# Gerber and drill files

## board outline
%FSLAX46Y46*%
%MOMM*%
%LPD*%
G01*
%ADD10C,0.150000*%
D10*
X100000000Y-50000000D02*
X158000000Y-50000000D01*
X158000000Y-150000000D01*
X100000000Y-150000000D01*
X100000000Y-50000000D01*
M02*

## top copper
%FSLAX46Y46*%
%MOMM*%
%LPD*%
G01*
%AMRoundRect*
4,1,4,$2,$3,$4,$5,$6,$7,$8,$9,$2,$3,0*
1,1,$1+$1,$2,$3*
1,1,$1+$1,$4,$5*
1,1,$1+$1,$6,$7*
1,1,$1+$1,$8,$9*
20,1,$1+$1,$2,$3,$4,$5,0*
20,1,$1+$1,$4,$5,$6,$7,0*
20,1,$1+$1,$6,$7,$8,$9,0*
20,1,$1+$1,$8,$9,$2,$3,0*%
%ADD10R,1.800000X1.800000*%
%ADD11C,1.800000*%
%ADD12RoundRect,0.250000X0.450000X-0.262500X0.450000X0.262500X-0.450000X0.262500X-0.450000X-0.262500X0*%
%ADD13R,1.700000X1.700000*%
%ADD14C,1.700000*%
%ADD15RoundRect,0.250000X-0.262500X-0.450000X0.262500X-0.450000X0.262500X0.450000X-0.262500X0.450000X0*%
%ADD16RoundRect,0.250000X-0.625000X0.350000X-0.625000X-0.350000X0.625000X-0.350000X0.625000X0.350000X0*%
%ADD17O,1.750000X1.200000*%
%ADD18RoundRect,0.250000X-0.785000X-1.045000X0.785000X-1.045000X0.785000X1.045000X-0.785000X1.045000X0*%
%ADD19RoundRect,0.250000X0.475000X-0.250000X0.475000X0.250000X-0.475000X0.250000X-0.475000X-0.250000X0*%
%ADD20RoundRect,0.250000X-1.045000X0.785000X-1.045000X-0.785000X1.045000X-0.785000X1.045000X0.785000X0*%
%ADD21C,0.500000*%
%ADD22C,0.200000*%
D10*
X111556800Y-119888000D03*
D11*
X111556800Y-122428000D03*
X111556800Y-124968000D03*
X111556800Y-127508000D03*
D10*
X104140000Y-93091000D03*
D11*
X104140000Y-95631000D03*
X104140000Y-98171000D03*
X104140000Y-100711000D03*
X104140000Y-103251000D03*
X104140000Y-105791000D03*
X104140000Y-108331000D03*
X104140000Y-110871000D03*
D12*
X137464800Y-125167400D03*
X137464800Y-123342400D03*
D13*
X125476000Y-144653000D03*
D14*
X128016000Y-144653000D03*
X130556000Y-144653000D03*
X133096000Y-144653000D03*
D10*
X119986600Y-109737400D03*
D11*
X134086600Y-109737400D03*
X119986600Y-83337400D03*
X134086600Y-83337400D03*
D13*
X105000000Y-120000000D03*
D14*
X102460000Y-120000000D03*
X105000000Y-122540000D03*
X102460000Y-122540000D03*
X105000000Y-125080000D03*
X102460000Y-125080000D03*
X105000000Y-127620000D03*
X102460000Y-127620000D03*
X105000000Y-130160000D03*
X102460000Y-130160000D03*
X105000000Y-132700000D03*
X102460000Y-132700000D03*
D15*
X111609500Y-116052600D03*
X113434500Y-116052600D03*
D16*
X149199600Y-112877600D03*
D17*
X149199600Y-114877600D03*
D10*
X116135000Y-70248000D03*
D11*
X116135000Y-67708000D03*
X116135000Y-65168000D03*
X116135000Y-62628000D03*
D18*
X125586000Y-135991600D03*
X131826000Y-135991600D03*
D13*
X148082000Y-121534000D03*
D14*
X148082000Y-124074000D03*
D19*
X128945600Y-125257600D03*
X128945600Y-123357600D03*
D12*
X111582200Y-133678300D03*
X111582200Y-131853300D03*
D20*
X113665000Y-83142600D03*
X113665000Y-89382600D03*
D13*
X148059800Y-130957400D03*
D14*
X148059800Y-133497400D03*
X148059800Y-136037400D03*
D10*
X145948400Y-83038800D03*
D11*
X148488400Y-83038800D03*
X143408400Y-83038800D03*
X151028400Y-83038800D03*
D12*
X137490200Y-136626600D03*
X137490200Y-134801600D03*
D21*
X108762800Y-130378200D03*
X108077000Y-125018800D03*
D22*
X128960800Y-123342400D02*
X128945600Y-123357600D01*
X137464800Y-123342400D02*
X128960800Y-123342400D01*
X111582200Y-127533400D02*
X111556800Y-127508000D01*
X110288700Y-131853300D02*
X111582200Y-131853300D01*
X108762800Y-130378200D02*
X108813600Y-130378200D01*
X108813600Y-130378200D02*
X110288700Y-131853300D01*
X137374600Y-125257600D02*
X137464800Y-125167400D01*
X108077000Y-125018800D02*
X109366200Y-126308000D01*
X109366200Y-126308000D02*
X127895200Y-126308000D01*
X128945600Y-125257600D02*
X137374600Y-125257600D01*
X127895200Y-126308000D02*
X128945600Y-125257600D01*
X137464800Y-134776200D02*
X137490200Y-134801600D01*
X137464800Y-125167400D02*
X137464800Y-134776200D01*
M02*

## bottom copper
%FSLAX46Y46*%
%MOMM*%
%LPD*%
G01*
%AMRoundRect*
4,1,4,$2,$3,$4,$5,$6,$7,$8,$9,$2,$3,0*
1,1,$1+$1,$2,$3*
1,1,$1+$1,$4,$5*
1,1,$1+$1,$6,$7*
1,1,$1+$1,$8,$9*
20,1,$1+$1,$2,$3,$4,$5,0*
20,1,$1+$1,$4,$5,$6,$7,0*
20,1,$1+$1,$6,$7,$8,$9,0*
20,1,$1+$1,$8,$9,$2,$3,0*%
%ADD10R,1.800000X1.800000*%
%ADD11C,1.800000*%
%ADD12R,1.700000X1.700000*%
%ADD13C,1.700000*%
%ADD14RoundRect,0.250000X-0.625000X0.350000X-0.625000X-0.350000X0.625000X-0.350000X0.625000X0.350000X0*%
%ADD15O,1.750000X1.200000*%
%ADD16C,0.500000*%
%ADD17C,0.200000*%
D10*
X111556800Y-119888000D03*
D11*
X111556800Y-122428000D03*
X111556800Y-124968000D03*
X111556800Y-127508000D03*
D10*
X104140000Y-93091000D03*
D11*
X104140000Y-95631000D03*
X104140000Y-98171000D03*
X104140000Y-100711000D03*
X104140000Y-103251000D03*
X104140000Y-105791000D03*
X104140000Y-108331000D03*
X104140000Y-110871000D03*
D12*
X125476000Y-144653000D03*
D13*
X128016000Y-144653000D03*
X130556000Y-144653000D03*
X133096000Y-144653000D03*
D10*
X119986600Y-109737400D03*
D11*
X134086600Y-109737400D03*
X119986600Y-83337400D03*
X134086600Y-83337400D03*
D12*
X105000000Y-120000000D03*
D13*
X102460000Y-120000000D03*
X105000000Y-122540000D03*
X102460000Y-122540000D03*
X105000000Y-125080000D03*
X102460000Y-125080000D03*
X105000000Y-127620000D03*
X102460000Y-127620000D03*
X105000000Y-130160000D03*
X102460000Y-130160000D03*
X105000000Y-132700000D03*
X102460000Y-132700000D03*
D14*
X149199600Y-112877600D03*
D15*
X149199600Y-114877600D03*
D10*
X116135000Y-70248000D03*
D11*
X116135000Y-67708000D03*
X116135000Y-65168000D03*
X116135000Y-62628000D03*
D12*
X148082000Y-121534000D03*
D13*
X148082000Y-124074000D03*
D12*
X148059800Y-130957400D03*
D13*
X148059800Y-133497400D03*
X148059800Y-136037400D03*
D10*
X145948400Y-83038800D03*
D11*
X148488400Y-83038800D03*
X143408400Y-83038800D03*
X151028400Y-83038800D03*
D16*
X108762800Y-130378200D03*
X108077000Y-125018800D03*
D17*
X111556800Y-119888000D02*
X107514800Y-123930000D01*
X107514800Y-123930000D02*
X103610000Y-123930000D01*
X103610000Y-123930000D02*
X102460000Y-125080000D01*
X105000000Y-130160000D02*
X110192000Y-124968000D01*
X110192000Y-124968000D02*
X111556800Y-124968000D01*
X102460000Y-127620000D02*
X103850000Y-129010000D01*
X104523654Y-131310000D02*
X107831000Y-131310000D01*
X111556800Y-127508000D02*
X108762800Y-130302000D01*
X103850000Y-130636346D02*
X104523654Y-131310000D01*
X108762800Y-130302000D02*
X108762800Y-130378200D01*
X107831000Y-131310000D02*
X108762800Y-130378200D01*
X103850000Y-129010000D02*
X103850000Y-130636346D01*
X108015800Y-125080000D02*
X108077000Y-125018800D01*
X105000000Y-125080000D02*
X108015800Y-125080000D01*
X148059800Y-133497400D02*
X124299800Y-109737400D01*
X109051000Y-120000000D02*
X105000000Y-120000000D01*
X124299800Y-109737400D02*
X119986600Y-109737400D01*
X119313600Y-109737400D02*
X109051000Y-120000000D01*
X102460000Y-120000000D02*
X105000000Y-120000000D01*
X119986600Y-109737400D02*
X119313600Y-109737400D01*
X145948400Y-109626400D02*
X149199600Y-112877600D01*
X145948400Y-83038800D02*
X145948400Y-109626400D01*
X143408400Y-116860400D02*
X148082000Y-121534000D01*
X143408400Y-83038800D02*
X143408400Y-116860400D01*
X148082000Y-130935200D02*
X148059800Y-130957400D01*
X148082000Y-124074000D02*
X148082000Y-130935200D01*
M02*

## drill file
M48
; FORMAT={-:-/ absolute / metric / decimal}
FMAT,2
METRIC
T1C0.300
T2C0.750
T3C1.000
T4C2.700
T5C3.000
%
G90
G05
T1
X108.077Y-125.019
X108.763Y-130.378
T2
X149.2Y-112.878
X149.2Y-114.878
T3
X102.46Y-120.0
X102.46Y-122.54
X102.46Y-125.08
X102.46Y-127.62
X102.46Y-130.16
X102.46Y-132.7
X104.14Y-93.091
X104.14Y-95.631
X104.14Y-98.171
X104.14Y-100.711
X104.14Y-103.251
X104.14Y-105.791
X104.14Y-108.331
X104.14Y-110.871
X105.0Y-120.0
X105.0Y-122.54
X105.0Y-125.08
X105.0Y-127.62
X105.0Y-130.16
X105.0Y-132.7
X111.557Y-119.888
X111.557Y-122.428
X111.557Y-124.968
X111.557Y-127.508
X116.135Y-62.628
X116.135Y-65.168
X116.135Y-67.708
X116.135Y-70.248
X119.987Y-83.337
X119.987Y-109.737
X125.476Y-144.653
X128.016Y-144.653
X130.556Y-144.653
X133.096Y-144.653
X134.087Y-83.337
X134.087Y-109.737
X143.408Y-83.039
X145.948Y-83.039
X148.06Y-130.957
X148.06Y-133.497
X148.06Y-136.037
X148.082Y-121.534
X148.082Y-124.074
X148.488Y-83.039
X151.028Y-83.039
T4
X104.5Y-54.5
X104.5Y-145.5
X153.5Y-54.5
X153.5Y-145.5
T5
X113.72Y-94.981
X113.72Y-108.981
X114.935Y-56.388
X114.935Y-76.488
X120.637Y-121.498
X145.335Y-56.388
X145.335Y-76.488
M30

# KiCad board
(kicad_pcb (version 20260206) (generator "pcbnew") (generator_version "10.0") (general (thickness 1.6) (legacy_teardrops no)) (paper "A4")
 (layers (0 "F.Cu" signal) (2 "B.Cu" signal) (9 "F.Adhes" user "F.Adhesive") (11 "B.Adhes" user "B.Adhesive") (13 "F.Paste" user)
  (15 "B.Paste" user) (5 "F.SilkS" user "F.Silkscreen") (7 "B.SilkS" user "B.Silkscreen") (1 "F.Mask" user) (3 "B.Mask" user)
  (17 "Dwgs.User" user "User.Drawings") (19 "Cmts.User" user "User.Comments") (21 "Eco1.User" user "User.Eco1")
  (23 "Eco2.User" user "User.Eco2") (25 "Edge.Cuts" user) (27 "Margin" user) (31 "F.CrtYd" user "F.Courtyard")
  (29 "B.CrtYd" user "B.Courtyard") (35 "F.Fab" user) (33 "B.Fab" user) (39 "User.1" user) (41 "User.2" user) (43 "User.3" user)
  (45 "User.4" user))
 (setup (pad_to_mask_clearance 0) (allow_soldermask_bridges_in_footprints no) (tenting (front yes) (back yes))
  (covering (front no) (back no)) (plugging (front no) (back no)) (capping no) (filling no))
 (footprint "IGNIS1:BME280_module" (layer "F.Cu") (at 116.6368 123.698)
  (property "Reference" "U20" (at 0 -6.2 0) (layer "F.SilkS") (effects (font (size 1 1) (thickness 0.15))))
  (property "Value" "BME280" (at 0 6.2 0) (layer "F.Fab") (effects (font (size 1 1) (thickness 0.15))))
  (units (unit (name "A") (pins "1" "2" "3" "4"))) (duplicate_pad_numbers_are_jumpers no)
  (pad "" np_thru_hole circle (at 4 -2.2) (size 3 3) (drill 3) (layers "*.Cu" "*.Mask"))
  (pad "1" thru_hole rect (at -5.08 -3.81) (size 1.8 1.8) (drill 1) (layers "*.Cu" "*.Mask") (remove_unused_layers no) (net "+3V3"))
  (pad "2" thru_hole circle (at -5.08 -1.27) (size 1.8 1.8) (drill 1) (layers "*.Cu" "*.Mask") (remove_unused_layers no) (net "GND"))
  (pad "3" thru_hole circle (at -5.08 1.27) (size 1.8 1.8) (drill 1) (layers "*.Cu" "*.Mask") (remove_unused_layers no) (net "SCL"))
  (pad "4" thru_hole circle (at -5.08 3.81) (size 1.8 1.8) (drill 1) (layers "*.Cu" "*.Mask") (remove_unused_layers no) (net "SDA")))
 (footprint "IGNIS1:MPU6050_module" (layer "F.Cu") (at 109.22 101.981)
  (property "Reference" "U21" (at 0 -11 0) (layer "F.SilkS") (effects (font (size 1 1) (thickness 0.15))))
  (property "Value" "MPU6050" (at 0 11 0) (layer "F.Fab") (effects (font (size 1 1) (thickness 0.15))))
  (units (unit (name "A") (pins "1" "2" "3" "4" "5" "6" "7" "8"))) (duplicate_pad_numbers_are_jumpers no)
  (pad "" np_thru_hole circle (at 4.5 -7) (size 3 3) (drill 3) (layers "*.Cu" "*.Mask"))
  (pad "" np_thru_hole circle (at 4.5 7) (size 3 3) (drill 3) (layers "*.Cu" "*.Mask"))
  (pad "1" thru_hole rect (at -5.08 -8.89) (size 1.8 1.8) (drill 1) (layers "*.Cu" "*.Mask") (remove_unused_layers no) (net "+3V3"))
  (pad "2" thru_hole circle (at -5.08 -6.35) (size 1.8 1.8) (drill 1) (layers "*.Cu" "*.Mask") (remove_unused_layers no) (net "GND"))
  (pad "3" thru_hole circle (at -5.08 -3.81) (size 1.8 1.8) (drill 1) (layers "*.Cu" "*.Mask") (remove_unused_layers no) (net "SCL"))
  (pad "4" thru_hole circle (at -5.08 -1.27) (size 1.8 1.8) (drill 1) (layers "*.Cu" "*.Mask") (remove_unused_layers no) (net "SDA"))
  (pad "5" thru_hole circle (at -5.08 1.27) (size 1.8 1.8) (drill 1) (layers "*.Cu" "*.Mask") (remove_unused_layers no)
   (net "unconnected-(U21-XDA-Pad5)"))
  (pad "6" thru_hole circle (at -5.08 3.81) (size 1.8 1.8) (drill 1) (layers "*.Cu" "*.Mask") (remove_unused_layers no)
   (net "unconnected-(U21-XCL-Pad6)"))
  (pad "7" thru_hole circle (at -5.08 6.35) (size 1.8 1.8) (drill 1) (layers "*.Cu" "*.Mask") (remove_unused_layers no) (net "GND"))
  (pad "8" thru_hole circle (at -5.08 8.89) (size 1.8 1.8) (drill 1) (layers "*.Cu" "*.Mask") (remove_unused_layers no) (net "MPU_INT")))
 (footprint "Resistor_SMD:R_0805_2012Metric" (layer "F.Cu") (at 137.4648 124.2549 90)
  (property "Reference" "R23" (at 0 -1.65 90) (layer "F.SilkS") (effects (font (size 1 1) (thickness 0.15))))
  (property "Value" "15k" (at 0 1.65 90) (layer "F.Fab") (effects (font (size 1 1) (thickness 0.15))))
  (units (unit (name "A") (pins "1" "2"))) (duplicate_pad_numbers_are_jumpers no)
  (pad "1" smd roundrect (at -0.9125 0 90) (size 1.025 1.4) (layers "F.Cu" "F.Mask" "F.Paste") (roundrect_rratio 0.243902) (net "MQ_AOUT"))
  (pad "2" smd roundrect (at 0.9125 0 90) (size 1.025 1.4) (layers "F.Cu" "F.Mask" "F.Paste") (roundrect_rratio 0.243902) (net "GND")))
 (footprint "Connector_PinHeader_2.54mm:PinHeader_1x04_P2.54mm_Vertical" (layer "F.Cu") (at 125.476 144.653 90)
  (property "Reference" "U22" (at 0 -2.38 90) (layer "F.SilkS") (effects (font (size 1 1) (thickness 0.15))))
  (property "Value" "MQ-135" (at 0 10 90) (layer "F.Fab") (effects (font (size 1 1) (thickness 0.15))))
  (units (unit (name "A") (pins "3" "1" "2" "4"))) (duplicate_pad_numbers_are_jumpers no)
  (pad "1" thru_hole rect (at 0 0 90) (size 1.7 1.7) (drill 1) (layers "*.Cu" "*.Mask") (remove_unused_layers no) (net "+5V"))
  (pad "2" thru_hole circle (at 0 2.54 90) (size 1.7 1.7) (drill 1) (layers "*.Cu" "*.Mask") (remove_unused_layers no) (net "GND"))
  (pad "3" thru_hole circle (at 0 5.08 90) (size 1.7 1.7) (drill 1) (layers "*.Cu" "*.Mask") (remove_unused_layers no)
   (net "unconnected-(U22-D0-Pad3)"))
  (pad "4" thru_hole circle (at 0 7.62 90) (size 1.7 1.7) (drill 1) (layers "*.Cu" "*.Mask") (remove_unused_layers no) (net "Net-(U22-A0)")))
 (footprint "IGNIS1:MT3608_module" (layer "F.Cu") (at 127.0366 96.5374 90)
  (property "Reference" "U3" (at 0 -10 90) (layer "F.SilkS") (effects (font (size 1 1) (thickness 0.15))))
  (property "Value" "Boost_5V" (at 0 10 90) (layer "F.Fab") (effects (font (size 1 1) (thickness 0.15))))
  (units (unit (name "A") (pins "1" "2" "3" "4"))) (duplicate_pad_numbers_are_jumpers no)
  (pad "1" thru_hole rect (at -13.2 -7.05 90) (size 1.8 1.8) (drill 1) (layers "*.Cu" "*.Mask") (remove_unused_layers no) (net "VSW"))
  (pad "2" thru_hole circle (at -13.2 7.05 90) (size 1.8 1.8) (drill 1) (layers "*.Cu" "*.Mask") (remove_unused_layers no) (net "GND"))
  (pad "3" thru_hole circle (at 13.2 -7.05 90) (size 1.8 1.8) (drill 1) (layers "*.Cu" "*.Mask") (remove_unused_layers no) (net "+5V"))
  (pad "4" thru_hole circle (at 13.2 7.05 90) (size 1.8 1.8) (drill 1) (layers "*.Cu" "*.Mask") (remove_unused_layers no) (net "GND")))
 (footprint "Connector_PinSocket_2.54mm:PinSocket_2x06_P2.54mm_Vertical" (layer "F.Cu") (at 105 120)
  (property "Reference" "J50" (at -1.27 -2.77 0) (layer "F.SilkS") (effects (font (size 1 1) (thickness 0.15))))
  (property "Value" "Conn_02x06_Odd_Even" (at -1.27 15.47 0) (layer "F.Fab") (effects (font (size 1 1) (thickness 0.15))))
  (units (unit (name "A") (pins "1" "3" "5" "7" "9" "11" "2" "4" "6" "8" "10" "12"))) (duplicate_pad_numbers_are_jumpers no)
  (pad "1" thru_hole rect (at 0 0) (size 1.7 1.7) (drill 1) (layers "*.Cu" "*.Mask") (remove_unused_layers no) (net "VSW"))
  (pad "2" thru_hole circle (at -2.54 0) (size 1.7 1.7) (drill 1) (layers "*.Cu" "*.Mask") (remove_unused_layers no) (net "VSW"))
  (pad "3" thru_hole circle (at 0 2.54) (size 1.7 1.7) (drill 1) (layers "*.Cu" "*.Mask") (remove_unused_layers no) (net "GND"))
  (pad "4" thru_hole circle (at -2.54 2.54) (size 1.7 1.7) (drill 1) (layers "*.Cu" "*.Mask") (remove_unused_layers no) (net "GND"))
  (pad "5" thru_hole circle (at 0 5.08) (size 1.7 1.7) (drill 1) (layers "*.Cu" "*.Mask") (remove_unused_layers no) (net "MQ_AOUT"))
  (pad "6" thru_hole circle (at -2.54 5.08) (size 1.7 1.7) (drill 1) (layers "*.Cu" "*.Mask") (remove_unused_layers no) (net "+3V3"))
  (pad "7" thru_hole circle (at 0 7.62) (size 1.7 1.7) (drill 1) (layers "*.Cu" "*.Mask") (remove_unused_layers no) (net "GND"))
  (pad "8" thru_hole circle (at -2.54 7.62) (size 1.7 1.7) (drill 1) (layers "*.Cu" "*.Mask") (remove_unused_layers no) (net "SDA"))
  (pad "9" thru_hole circle (at 0 10.16) (size 1.7 1.7) (drill 1) (layers "*.Cu" "*.Mask") (remove_unused_layers no) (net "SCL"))
  (pad "10" thru_hole circle (at -2.54 10.16) (size 1.7 1.7) (drill 1) (layers "*.Cu" "*.Mask") (remove_unused_layers no) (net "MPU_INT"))
  (pad "11" thru_hole circle (at 0 12.7) (size 1.7 1.7) (drill 1) (layers "*.Cu" "*.Mask") (remove_unused_layers no) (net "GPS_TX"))
  (pad "12" thru_hole circle (at -2.54 12.7) (size 1.7 1.7) (drill 1) (layers "*.Cu" "*.Mask") (remove_unused_layers no) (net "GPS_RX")))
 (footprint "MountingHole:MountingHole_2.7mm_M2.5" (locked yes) (layer "F.Cu") (at 104.5 145.5)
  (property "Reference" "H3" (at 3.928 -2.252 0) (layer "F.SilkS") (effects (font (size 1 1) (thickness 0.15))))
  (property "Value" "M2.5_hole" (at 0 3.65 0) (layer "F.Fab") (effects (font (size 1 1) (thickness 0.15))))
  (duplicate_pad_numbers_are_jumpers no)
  (pad "" np_thru_hole circle (at 0 0) (size 2.7 2.7) (drill 2.7) (layers "*.Cu" "*.Mask")))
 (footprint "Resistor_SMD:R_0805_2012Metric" (layer "F.Cu") (at 112.522 116.0526)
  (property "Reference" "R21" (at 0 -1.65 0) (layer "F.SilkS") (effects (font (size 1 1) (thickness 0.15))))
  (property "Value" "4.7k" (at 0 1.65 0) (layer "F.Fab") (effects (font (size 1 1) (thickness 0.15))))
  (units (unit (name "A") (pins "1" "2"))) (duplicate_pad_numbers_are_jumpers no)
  (pad "1" smd roundrect (at -0.9125 0) (size 1.025 1.4) (layers "F.Cu" "F.Mask" "F.Paste") (roundrect_rratio 0.243902) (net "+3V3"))
  (pad "2" smd roundrect (at 0.9125 0) (size 1.025 1.4) (layers "F.Cu" "F.Mask" "F.Paste") (roundrect_rratio 0.243902) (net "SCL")))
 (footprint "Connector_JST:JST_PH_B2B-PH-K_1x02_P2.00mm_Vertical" (layer "F.Cu") (at 149.1996 112.8776 -90)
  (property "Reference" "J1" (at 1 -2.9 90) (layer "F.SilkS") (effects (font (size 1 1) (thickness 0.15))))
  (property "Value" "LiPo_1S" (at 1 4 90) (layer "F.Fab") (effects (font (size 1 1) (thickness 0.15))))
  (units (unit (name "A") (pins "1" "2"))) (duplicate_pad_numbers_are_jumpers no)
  (pad "1" thru_hole roundrect (at 0 0 270) (size 1.2 1.75) (drill 0.75) (layers "*.Cu" "*.Mask") (remove_unused_layers no)
   (roundrect_rratio 0.208333) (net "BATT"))
  (pad "2" thru_hole oval (at 2 0 270) (size 1.2 1.75) (drill 0.75) (layers "*.Cu" "*.Mask") (remove_unused_layers no) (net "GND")))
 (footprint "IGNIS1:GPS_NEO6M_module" (layer "F.Cu") (at 130.135 66.438)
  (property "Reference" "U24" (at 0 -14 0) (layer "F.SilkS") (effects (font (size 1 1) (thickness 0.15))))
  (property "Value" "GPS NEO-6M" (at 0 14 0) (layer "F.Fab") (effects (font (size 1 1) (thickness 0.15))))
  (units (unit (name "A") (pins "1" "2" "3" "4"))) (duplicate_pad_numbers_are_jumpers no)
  (pad "" np_thru_hole circle (at -15.2 -10.05) (size 3 3) (drill 3) (layers "*.Cu" "*.Mask"))
  (pad "" np_thru_hole circle (at -15.2 10.05) (size 3 3) (drill 3) (layers "*.Cu" "*.Mask"))
  (pad "" np_thru_hole circle (at 15.2 -10.05) (size 3 3) (drill 3) (layers "*.Cu" "*.Mask"))
  (pad "" np_thru_hole circle (at 15.2 10.05) (size 3 3) (drill 3) (layers "*.Cu" "*.Mask"))
  (pad "1" thru_hole rect (at -14 3.81) (size 1.8 1.8) (drill 1) (layers "*.Cu" "*.Mask") (remove_unused_layers no) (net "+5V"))
  (pad "2" thru_hole circle (at -14 1.27) (size 1.8 1.8) (drill 1) (layers "*.Cu" "*.Mask") (remove_unused_layers no) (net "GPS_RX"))
  (pad "3" thru_hole circle (at -14 -1.27) (size 1.8 1.8) (drill 1) (layers "*.Cu" "*.Mask") (remove_unused_layers no) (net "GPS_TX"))
  (pad "4" thru_hole circle (at -14 -3.81) (size 1.8 1.8) (drill 1) (layers "*.Cu" "*.Mask") (remove_unused_layers no) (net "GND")))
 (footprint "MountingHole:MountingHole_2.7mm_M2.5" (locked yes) (layer "F.Cu") (at 153.5 145.5)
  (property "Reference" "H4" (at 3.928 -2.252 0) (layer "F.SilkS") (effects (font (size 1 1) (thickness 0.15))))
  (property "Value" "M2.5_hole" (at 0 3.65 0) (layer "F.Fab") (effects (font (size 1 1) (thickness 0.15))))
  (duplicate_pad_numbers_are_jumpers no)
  (pad "" np_thru_hole circle (at 0 0) (size 2.7 2.7) (drill 2.7) (layers "*.Cu" "*.Mask")))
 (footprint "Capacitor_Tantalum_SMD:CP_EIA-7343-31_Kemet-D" (layer "F.Cu") (at 128.706 135.9916)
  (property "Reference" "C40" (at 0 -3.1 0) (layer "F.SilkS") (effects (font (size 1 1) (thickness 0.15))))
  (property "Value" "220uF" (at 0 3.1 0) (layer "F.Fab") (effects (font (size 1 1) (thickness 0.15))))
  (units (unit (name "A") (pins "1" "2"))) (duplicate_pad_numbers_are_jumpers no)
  (pad "1" smd roundrect (at -3.12 0) (size 2.07 2.59) (layers "F.Cu" "F.Mask" "F.Paste") (roundrect_rratio 0.120773) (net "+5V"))
  (pad "2" smd roundrect (at 3.12 0) (size 2.07 2.59) (layers "F.Cu" "F.Mask" "F.Paste") (roundrect_rratio 0.120773) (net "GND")))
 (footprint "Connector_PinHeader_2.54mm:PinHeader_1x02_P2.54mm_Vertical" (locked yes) (layer "F.Cu") (at 148.082 121.534)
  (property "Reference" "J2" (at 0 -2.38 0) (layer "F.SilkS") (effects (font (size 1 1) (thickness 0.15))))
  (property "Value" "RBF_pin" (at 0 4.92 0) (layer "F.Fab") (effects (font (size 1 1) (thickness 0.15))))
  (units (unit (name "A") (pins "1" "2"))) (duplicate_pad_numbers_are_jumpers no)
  (pad "1" thru_hole rect (at 0 0) (size 1.7 1.7) (drill 1) (layers "*.Cu" "*.Mask") (remove_unused_layers no) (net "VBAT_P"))
  (pad "2" thru_hole circle (at 0 2.54) (size 1.7 1.7) (drill 1) (layers "*.Cu" "*.Mask") (remove_unused_layers no) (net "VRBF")))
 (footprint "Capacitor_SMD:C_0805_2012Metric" (layer "F.Cu") (at 128.9456 124.3076 90)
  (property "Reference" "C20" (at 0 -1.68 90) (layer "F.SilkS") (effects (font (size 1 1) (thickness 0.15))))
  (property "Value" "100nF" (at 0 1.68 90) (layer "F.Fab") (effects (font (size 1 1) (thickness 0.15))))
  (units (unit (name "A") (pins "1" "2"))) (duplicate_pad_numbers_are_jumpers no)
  (pad "1" smd roundrect (at -0.95 0 90) (size 1 1.45) (layers "F.Cu" "F.Mask" "F.Paste") (roundrect_rratio 0.25) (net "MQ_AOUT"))
  (pad "2" smd roundrect (at 0.95 0 90) (size 1 1.45) (layers "F.Cu" "F.Mask" "F.Paste") (roundrect_rratio 0.25) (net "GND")))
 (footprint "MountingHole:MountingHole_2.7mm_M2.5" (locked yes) (layer "F.Cu") (at 153.5 54.5)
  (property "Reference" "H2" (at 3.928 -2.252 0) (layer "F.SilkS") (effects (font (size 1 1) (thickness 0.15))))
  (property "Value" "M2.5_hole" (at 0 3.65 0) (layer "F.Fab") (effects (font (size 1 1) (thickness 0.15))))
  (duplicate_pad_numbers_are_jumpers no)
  (pad "" np_thru_hole circle (at 0 0) (size 2.7 2.7) (drill 2.7) (layers "*.Cu" "*.Mask")))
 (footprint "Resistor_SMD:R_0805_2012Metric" (layer "F.Cu") (at 111.5822 132.7658 90)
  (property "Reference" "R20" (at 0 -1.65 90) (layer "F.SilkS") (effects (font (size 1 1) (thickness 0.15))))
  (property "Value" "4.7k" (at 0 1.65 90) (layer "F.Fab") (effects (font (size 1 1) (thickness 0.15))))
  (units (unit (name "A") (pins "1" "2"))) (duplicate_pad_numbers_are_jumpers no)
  (pad "1" smd roundrect (at -0.9125 0 90) (size 1.025 1.4) (layers "F.Cu" "F.Mask" "F.Paste") (roundrect_rratio 0.243902) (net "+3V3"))
  (pad "2" smd roundrect (at 0.9125 0 90) (size 1.025 1.4) (layers "F.Cu" "F.Mask" "F.Paste") (roundrect_rratio 0.243902) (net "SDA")))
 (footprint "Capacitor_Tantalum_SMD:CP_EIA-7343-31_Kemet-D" (layer "F.Cu") (at 113.665 86.2626 -90)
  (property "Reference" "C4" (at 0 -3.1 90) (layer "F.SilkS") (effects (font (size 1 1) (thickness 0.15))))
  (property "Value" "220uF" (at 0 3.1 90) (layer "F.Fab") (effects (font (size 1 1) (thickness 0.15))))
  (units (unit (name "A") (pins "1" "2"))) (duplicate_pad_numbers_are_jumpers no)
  (pad "1" smd roundrect (at -3.12 0 270) (size 2.07 2.59) (layers "F.Cu" "F.Mask" "F.Paste") (roundrect_rratio 0.120773) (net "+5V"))
  (pad "2" smd roundrect (at 3.12 0 270) (size 2.07 2.59) (layers "F.Cu" "F.Mask" "F.Paste") (roundrect_rratio 0.120773) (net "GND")))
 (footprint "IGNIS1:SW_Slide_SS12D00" (layer "F.Cu") (at 148.0598 133.4974 -90)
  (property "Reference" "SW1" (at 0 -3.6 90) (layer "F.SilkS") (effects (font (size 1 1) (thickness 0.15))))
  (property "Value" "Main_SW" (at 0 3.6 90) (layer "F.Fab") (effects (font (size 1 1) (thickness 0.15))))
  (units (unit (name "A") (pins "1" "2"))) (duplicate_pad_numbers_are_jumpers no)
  (pad "1" thru_hole rect (at -2.54 0 270) (size 1.7 1.7) (drill 1) (layers "*.Cu" "*.Mask") (remove_unused_layers no) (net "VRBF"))
  (pad "2" thru_hole circle (at 0 0 270) (size 1.7 1.7) (drill 1) (layers "*.Cu" "*.Mask") (remove_unused_layers no) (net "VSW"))
  (pad "3" thru_hole circle (at 2.54 0 270) (size 1.7 1.7) (drill 1) (layers "*.Cu" "*.Mask") (remove_unused_layers no)))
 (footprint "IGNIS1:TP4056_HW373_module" (layer "F.Cu") (at 147.2184 94.5388 90)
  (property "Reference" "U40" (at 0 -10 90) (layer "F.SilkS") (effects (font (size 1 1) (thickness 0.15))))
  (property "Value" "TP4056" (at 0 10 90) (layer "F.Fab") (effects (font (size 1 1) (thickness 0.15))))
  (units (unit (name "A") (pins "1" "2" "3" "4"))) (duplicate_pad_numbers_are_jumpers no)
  (pad "1" thru_hole rect (at 11.5 -1.27 90) (size 1.8 1.8) (drill 1) (layers "*.Cu" "*.Mask") (remove_unused_layers no) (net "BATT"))
  (pad "2" thru_hole circle (at 11.5 1.27 90) (size 1.8 1.8) (drill 1) (layers "*.Cu" "*.Mask") (remove_unused_layers no) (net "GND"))
  (pad "3" thru_hole circle (at 11.5 -3.81 90) (size 1.8 1.8) (drill 1) (layers "*.Cu" "*.Mask") (remove_unused_layers no) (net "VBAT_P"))
  (pad "4" thru_hole circle (at 11.5 3.81 90) (size 1.8 1.8) (drill 1) (layers "*.Cu" "*.Mask") (remove_unused_layers no) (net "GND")))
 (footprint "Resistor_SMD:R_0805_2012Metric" (layer "F.Cu") (at 137.4902 135.7141 90)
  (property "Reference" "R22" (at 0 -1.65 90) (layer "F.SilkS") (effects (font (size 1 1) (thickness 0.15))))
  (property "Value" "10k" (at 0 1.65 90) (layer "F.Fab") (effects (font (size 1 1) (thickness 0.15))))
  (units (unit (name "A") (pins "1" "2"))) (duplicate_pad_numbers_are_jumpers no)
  (pad "1" smd roundrect (at -0.9125 0 90) (size 1.025 1.4) (layers "F.Cu" "F.Mask" "F.Paste") (roundrect_rratio 0.243902)
   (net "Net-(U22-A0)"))
  (pad "2" smd roundrect (at 0.9125 0 90) (size 1.025 1.4) (layers "F.Cu" "F.Mask" "F.Paste") (roundrect_rratio 0.243902) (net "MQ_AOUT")))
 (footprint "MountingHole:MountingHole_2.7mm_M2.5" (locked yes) (layer "F.Cu") (at 104.5 54.5)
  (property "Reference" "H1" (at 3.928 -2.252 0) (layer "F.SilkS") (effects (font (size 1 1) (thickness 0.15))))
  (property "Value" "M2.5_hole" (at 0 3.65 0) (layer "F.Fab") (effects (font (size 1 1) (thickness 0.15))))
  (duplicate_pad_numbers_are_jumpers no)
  (pad "" np_thru_hole circle (at 0 0) (size 2.7 2.7) (drill 2.7) (layers "*.Cu" "*.Mask")))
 (gr_rect (start 100 50) (end 158 150) (stroke (width 0.15) (type solid)) (fill no) (locked yes) (layer "Edge.Cuts"))
 (segment (start 111.5568 119.888) (end 107.5148 123.93) (width 0.2) (layer "B.Cu") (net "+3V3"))
 (segment (start 107.5148 123.93) (end 103.61 123.93) (width 0.2) (layer "B.Cu") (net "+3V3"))
 (segment (start 103.61 123.93) (end 102.46 125.08) (width 0.2) (layer "B.Cu") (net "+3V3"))
 (segment (start 128.9608 123.3424) (end 128.9456 123.3576) (width 0.2) (layer "F.Cu") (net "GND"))
 (segment (start 137.4648 123.3424) (end 128.9608 123.3424) (width 0.2) (layer "F.Cu") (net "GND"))
 (segment (start 105 130.16) (end 110.192 124.968) (width 0.2) (layer "B.Cu") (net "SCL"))
 (segment (start 110.192 124.968) (end 111.5568 124.968) (width 0.2) (layer "B.Cu") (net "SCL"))
 (segment (start 111.5822 127.5334) (end 111.5568 127.508) (width 0.2) (layer "F.Cu") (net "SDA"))
 (segment (start 110.2887 131.8533) (end 111.5822 131.8533) (width 0.2) (layer "F.Cu") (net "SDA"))
 (segment (start 108.7628 130.3782) (end 108.8136 130.3782) (width 0.2) (layer "F.Cu") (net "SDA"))
 (segment (start 108.8136 130.3782) (end 110.2887 131.8533) (width 0.2) (layer "F.Cu") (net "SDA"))
 (via (at 108.7628 130.3782) (size 0.5) (drill 0.3) (layers "F.Cu" "B.Cu") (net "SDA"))
 (segment (start 102.46 127.62) (end 103.85 129.01) (width 0.2) (layer "B.Cu") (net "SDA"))
 (segment (start 104.523654 131.31) (end 107.831 131.31) (width 0.2) (layer "B.Cu") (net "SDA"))
 (segment (start 111.5568 127.508) (end 108.7628 130.302) (width 0.2) (layer "B.Cu") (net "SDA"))
 (segment (start 103.85 130.636346) (end 104.523654 131.31) (width 0.2) (layer "B.Cu") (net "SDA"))
 (segment (start 108.7628 130.302) (end 108.7628 130.3782) (width 0.2) (layer "B.Cu") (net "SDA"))
 (segment (start 107.831 131.31) (end 108.7628 130.3782) (width 0.2) (layer "B.Cu") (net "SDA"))
 (segment (start 103.85 129.01) (end 103.85 130.636346) (width 0.2) (layer "B.Cu") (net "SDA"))
 (segment (start 137.3746 125.2576) (end 137.4648 125.1674) (width 0.2) (layer "F.Cu") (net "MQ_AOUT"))
 (segment (start 108.077 125.0188) (end 109.3662 126.308) (width 0.2) (layer "F.Cu") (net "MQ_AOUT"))
 (segment (start 109.3662 126.308) (end 127.8952 126.308) (width 0.2) (layer "F.Cu") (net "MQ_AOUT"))
 (segment (start 128.9456 125.2576) (end 137.3746 125.2576) (width 0.2) (layer "F.Cu") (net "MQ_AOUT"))
 (segment (start 127.8952 126.308) (end 128.9456 125.2576) (width 0.2) (layer "F.Cu") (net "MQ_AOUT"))
 (segment (start 137.4648 134.7762) (end 137.4902 134.8016) (width 0.2) (layer "F.Cu") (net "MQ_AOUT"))
 (segment (start 137.4648 125.1674) (end 137.4648 134.7762) (width 0.2) (layer "F.Cu") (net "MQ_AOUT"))
 (via (at 108.077 125.0188) (size 0.5) (drill 0.3) (layers "F.Cu" "B.Cu") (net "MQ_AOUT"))
 (segment (start 108.0158 125.08) (end 108.077 125.0188) (width 0.2) (layer "B.Cu") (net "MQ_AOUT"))
 (segment (start 105 125.08) (end 108.0158 125.08) (width 0.2) (layer "B.Cu") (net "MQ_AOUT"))
 (segment (start 148.0598 133.4974) (end 124.2998 109.7374) (width 0.2) (layer "B.Cu") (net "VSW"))
 (segment (start 109.051 120) (end 105 120) (width 0.2) (layer "B.Cu") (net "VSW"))
 (segment (start 124.2998 109.7374) (end 119.9866 109.7374) (width 0.2) (layer "B.Cu") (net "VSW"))
 (segment (start 119.3136 109.7374) (end 109.051 120) (width 0.2) (layer "B.Cu") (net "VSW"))
 (segment (start 102.46 120) (end 105 120) (width 0.2) (layer "B.Cu") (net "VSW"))
 (segment (start 119.9866 109.7374) (end 119.3136 109.7374) (width 0.2) (layer "B.Cu") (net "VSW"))
 (segment (start 145.9484 109.6264) (end 149.1996 112.8776) (width 0.2) (layer "B.Cu") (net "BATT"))
 (segment (start 145.9484 83.0388) (end 145.9484 109.6264) (width 0.2) (layer "B.Cu") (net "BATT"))
 (segment (start 143.4084 116.8604) (end 148.082 121.534) (width 0.2) (layer "B.Cu") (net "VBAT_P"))
 (segment (start 143.4084 83.0388) (end 143.4084 116.8604) (width 0.2) (layer "B.Cu") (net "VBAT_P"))
 (segment (start 148.082 130.9352) (end 148.0598 130.9574) (width 0.2) (layer "B.Cu") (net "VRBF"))
 (segment (start 148.082 124.074) (end 148.082 130.9352) (width 0.2) (layer "B.Cu") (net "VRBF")))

